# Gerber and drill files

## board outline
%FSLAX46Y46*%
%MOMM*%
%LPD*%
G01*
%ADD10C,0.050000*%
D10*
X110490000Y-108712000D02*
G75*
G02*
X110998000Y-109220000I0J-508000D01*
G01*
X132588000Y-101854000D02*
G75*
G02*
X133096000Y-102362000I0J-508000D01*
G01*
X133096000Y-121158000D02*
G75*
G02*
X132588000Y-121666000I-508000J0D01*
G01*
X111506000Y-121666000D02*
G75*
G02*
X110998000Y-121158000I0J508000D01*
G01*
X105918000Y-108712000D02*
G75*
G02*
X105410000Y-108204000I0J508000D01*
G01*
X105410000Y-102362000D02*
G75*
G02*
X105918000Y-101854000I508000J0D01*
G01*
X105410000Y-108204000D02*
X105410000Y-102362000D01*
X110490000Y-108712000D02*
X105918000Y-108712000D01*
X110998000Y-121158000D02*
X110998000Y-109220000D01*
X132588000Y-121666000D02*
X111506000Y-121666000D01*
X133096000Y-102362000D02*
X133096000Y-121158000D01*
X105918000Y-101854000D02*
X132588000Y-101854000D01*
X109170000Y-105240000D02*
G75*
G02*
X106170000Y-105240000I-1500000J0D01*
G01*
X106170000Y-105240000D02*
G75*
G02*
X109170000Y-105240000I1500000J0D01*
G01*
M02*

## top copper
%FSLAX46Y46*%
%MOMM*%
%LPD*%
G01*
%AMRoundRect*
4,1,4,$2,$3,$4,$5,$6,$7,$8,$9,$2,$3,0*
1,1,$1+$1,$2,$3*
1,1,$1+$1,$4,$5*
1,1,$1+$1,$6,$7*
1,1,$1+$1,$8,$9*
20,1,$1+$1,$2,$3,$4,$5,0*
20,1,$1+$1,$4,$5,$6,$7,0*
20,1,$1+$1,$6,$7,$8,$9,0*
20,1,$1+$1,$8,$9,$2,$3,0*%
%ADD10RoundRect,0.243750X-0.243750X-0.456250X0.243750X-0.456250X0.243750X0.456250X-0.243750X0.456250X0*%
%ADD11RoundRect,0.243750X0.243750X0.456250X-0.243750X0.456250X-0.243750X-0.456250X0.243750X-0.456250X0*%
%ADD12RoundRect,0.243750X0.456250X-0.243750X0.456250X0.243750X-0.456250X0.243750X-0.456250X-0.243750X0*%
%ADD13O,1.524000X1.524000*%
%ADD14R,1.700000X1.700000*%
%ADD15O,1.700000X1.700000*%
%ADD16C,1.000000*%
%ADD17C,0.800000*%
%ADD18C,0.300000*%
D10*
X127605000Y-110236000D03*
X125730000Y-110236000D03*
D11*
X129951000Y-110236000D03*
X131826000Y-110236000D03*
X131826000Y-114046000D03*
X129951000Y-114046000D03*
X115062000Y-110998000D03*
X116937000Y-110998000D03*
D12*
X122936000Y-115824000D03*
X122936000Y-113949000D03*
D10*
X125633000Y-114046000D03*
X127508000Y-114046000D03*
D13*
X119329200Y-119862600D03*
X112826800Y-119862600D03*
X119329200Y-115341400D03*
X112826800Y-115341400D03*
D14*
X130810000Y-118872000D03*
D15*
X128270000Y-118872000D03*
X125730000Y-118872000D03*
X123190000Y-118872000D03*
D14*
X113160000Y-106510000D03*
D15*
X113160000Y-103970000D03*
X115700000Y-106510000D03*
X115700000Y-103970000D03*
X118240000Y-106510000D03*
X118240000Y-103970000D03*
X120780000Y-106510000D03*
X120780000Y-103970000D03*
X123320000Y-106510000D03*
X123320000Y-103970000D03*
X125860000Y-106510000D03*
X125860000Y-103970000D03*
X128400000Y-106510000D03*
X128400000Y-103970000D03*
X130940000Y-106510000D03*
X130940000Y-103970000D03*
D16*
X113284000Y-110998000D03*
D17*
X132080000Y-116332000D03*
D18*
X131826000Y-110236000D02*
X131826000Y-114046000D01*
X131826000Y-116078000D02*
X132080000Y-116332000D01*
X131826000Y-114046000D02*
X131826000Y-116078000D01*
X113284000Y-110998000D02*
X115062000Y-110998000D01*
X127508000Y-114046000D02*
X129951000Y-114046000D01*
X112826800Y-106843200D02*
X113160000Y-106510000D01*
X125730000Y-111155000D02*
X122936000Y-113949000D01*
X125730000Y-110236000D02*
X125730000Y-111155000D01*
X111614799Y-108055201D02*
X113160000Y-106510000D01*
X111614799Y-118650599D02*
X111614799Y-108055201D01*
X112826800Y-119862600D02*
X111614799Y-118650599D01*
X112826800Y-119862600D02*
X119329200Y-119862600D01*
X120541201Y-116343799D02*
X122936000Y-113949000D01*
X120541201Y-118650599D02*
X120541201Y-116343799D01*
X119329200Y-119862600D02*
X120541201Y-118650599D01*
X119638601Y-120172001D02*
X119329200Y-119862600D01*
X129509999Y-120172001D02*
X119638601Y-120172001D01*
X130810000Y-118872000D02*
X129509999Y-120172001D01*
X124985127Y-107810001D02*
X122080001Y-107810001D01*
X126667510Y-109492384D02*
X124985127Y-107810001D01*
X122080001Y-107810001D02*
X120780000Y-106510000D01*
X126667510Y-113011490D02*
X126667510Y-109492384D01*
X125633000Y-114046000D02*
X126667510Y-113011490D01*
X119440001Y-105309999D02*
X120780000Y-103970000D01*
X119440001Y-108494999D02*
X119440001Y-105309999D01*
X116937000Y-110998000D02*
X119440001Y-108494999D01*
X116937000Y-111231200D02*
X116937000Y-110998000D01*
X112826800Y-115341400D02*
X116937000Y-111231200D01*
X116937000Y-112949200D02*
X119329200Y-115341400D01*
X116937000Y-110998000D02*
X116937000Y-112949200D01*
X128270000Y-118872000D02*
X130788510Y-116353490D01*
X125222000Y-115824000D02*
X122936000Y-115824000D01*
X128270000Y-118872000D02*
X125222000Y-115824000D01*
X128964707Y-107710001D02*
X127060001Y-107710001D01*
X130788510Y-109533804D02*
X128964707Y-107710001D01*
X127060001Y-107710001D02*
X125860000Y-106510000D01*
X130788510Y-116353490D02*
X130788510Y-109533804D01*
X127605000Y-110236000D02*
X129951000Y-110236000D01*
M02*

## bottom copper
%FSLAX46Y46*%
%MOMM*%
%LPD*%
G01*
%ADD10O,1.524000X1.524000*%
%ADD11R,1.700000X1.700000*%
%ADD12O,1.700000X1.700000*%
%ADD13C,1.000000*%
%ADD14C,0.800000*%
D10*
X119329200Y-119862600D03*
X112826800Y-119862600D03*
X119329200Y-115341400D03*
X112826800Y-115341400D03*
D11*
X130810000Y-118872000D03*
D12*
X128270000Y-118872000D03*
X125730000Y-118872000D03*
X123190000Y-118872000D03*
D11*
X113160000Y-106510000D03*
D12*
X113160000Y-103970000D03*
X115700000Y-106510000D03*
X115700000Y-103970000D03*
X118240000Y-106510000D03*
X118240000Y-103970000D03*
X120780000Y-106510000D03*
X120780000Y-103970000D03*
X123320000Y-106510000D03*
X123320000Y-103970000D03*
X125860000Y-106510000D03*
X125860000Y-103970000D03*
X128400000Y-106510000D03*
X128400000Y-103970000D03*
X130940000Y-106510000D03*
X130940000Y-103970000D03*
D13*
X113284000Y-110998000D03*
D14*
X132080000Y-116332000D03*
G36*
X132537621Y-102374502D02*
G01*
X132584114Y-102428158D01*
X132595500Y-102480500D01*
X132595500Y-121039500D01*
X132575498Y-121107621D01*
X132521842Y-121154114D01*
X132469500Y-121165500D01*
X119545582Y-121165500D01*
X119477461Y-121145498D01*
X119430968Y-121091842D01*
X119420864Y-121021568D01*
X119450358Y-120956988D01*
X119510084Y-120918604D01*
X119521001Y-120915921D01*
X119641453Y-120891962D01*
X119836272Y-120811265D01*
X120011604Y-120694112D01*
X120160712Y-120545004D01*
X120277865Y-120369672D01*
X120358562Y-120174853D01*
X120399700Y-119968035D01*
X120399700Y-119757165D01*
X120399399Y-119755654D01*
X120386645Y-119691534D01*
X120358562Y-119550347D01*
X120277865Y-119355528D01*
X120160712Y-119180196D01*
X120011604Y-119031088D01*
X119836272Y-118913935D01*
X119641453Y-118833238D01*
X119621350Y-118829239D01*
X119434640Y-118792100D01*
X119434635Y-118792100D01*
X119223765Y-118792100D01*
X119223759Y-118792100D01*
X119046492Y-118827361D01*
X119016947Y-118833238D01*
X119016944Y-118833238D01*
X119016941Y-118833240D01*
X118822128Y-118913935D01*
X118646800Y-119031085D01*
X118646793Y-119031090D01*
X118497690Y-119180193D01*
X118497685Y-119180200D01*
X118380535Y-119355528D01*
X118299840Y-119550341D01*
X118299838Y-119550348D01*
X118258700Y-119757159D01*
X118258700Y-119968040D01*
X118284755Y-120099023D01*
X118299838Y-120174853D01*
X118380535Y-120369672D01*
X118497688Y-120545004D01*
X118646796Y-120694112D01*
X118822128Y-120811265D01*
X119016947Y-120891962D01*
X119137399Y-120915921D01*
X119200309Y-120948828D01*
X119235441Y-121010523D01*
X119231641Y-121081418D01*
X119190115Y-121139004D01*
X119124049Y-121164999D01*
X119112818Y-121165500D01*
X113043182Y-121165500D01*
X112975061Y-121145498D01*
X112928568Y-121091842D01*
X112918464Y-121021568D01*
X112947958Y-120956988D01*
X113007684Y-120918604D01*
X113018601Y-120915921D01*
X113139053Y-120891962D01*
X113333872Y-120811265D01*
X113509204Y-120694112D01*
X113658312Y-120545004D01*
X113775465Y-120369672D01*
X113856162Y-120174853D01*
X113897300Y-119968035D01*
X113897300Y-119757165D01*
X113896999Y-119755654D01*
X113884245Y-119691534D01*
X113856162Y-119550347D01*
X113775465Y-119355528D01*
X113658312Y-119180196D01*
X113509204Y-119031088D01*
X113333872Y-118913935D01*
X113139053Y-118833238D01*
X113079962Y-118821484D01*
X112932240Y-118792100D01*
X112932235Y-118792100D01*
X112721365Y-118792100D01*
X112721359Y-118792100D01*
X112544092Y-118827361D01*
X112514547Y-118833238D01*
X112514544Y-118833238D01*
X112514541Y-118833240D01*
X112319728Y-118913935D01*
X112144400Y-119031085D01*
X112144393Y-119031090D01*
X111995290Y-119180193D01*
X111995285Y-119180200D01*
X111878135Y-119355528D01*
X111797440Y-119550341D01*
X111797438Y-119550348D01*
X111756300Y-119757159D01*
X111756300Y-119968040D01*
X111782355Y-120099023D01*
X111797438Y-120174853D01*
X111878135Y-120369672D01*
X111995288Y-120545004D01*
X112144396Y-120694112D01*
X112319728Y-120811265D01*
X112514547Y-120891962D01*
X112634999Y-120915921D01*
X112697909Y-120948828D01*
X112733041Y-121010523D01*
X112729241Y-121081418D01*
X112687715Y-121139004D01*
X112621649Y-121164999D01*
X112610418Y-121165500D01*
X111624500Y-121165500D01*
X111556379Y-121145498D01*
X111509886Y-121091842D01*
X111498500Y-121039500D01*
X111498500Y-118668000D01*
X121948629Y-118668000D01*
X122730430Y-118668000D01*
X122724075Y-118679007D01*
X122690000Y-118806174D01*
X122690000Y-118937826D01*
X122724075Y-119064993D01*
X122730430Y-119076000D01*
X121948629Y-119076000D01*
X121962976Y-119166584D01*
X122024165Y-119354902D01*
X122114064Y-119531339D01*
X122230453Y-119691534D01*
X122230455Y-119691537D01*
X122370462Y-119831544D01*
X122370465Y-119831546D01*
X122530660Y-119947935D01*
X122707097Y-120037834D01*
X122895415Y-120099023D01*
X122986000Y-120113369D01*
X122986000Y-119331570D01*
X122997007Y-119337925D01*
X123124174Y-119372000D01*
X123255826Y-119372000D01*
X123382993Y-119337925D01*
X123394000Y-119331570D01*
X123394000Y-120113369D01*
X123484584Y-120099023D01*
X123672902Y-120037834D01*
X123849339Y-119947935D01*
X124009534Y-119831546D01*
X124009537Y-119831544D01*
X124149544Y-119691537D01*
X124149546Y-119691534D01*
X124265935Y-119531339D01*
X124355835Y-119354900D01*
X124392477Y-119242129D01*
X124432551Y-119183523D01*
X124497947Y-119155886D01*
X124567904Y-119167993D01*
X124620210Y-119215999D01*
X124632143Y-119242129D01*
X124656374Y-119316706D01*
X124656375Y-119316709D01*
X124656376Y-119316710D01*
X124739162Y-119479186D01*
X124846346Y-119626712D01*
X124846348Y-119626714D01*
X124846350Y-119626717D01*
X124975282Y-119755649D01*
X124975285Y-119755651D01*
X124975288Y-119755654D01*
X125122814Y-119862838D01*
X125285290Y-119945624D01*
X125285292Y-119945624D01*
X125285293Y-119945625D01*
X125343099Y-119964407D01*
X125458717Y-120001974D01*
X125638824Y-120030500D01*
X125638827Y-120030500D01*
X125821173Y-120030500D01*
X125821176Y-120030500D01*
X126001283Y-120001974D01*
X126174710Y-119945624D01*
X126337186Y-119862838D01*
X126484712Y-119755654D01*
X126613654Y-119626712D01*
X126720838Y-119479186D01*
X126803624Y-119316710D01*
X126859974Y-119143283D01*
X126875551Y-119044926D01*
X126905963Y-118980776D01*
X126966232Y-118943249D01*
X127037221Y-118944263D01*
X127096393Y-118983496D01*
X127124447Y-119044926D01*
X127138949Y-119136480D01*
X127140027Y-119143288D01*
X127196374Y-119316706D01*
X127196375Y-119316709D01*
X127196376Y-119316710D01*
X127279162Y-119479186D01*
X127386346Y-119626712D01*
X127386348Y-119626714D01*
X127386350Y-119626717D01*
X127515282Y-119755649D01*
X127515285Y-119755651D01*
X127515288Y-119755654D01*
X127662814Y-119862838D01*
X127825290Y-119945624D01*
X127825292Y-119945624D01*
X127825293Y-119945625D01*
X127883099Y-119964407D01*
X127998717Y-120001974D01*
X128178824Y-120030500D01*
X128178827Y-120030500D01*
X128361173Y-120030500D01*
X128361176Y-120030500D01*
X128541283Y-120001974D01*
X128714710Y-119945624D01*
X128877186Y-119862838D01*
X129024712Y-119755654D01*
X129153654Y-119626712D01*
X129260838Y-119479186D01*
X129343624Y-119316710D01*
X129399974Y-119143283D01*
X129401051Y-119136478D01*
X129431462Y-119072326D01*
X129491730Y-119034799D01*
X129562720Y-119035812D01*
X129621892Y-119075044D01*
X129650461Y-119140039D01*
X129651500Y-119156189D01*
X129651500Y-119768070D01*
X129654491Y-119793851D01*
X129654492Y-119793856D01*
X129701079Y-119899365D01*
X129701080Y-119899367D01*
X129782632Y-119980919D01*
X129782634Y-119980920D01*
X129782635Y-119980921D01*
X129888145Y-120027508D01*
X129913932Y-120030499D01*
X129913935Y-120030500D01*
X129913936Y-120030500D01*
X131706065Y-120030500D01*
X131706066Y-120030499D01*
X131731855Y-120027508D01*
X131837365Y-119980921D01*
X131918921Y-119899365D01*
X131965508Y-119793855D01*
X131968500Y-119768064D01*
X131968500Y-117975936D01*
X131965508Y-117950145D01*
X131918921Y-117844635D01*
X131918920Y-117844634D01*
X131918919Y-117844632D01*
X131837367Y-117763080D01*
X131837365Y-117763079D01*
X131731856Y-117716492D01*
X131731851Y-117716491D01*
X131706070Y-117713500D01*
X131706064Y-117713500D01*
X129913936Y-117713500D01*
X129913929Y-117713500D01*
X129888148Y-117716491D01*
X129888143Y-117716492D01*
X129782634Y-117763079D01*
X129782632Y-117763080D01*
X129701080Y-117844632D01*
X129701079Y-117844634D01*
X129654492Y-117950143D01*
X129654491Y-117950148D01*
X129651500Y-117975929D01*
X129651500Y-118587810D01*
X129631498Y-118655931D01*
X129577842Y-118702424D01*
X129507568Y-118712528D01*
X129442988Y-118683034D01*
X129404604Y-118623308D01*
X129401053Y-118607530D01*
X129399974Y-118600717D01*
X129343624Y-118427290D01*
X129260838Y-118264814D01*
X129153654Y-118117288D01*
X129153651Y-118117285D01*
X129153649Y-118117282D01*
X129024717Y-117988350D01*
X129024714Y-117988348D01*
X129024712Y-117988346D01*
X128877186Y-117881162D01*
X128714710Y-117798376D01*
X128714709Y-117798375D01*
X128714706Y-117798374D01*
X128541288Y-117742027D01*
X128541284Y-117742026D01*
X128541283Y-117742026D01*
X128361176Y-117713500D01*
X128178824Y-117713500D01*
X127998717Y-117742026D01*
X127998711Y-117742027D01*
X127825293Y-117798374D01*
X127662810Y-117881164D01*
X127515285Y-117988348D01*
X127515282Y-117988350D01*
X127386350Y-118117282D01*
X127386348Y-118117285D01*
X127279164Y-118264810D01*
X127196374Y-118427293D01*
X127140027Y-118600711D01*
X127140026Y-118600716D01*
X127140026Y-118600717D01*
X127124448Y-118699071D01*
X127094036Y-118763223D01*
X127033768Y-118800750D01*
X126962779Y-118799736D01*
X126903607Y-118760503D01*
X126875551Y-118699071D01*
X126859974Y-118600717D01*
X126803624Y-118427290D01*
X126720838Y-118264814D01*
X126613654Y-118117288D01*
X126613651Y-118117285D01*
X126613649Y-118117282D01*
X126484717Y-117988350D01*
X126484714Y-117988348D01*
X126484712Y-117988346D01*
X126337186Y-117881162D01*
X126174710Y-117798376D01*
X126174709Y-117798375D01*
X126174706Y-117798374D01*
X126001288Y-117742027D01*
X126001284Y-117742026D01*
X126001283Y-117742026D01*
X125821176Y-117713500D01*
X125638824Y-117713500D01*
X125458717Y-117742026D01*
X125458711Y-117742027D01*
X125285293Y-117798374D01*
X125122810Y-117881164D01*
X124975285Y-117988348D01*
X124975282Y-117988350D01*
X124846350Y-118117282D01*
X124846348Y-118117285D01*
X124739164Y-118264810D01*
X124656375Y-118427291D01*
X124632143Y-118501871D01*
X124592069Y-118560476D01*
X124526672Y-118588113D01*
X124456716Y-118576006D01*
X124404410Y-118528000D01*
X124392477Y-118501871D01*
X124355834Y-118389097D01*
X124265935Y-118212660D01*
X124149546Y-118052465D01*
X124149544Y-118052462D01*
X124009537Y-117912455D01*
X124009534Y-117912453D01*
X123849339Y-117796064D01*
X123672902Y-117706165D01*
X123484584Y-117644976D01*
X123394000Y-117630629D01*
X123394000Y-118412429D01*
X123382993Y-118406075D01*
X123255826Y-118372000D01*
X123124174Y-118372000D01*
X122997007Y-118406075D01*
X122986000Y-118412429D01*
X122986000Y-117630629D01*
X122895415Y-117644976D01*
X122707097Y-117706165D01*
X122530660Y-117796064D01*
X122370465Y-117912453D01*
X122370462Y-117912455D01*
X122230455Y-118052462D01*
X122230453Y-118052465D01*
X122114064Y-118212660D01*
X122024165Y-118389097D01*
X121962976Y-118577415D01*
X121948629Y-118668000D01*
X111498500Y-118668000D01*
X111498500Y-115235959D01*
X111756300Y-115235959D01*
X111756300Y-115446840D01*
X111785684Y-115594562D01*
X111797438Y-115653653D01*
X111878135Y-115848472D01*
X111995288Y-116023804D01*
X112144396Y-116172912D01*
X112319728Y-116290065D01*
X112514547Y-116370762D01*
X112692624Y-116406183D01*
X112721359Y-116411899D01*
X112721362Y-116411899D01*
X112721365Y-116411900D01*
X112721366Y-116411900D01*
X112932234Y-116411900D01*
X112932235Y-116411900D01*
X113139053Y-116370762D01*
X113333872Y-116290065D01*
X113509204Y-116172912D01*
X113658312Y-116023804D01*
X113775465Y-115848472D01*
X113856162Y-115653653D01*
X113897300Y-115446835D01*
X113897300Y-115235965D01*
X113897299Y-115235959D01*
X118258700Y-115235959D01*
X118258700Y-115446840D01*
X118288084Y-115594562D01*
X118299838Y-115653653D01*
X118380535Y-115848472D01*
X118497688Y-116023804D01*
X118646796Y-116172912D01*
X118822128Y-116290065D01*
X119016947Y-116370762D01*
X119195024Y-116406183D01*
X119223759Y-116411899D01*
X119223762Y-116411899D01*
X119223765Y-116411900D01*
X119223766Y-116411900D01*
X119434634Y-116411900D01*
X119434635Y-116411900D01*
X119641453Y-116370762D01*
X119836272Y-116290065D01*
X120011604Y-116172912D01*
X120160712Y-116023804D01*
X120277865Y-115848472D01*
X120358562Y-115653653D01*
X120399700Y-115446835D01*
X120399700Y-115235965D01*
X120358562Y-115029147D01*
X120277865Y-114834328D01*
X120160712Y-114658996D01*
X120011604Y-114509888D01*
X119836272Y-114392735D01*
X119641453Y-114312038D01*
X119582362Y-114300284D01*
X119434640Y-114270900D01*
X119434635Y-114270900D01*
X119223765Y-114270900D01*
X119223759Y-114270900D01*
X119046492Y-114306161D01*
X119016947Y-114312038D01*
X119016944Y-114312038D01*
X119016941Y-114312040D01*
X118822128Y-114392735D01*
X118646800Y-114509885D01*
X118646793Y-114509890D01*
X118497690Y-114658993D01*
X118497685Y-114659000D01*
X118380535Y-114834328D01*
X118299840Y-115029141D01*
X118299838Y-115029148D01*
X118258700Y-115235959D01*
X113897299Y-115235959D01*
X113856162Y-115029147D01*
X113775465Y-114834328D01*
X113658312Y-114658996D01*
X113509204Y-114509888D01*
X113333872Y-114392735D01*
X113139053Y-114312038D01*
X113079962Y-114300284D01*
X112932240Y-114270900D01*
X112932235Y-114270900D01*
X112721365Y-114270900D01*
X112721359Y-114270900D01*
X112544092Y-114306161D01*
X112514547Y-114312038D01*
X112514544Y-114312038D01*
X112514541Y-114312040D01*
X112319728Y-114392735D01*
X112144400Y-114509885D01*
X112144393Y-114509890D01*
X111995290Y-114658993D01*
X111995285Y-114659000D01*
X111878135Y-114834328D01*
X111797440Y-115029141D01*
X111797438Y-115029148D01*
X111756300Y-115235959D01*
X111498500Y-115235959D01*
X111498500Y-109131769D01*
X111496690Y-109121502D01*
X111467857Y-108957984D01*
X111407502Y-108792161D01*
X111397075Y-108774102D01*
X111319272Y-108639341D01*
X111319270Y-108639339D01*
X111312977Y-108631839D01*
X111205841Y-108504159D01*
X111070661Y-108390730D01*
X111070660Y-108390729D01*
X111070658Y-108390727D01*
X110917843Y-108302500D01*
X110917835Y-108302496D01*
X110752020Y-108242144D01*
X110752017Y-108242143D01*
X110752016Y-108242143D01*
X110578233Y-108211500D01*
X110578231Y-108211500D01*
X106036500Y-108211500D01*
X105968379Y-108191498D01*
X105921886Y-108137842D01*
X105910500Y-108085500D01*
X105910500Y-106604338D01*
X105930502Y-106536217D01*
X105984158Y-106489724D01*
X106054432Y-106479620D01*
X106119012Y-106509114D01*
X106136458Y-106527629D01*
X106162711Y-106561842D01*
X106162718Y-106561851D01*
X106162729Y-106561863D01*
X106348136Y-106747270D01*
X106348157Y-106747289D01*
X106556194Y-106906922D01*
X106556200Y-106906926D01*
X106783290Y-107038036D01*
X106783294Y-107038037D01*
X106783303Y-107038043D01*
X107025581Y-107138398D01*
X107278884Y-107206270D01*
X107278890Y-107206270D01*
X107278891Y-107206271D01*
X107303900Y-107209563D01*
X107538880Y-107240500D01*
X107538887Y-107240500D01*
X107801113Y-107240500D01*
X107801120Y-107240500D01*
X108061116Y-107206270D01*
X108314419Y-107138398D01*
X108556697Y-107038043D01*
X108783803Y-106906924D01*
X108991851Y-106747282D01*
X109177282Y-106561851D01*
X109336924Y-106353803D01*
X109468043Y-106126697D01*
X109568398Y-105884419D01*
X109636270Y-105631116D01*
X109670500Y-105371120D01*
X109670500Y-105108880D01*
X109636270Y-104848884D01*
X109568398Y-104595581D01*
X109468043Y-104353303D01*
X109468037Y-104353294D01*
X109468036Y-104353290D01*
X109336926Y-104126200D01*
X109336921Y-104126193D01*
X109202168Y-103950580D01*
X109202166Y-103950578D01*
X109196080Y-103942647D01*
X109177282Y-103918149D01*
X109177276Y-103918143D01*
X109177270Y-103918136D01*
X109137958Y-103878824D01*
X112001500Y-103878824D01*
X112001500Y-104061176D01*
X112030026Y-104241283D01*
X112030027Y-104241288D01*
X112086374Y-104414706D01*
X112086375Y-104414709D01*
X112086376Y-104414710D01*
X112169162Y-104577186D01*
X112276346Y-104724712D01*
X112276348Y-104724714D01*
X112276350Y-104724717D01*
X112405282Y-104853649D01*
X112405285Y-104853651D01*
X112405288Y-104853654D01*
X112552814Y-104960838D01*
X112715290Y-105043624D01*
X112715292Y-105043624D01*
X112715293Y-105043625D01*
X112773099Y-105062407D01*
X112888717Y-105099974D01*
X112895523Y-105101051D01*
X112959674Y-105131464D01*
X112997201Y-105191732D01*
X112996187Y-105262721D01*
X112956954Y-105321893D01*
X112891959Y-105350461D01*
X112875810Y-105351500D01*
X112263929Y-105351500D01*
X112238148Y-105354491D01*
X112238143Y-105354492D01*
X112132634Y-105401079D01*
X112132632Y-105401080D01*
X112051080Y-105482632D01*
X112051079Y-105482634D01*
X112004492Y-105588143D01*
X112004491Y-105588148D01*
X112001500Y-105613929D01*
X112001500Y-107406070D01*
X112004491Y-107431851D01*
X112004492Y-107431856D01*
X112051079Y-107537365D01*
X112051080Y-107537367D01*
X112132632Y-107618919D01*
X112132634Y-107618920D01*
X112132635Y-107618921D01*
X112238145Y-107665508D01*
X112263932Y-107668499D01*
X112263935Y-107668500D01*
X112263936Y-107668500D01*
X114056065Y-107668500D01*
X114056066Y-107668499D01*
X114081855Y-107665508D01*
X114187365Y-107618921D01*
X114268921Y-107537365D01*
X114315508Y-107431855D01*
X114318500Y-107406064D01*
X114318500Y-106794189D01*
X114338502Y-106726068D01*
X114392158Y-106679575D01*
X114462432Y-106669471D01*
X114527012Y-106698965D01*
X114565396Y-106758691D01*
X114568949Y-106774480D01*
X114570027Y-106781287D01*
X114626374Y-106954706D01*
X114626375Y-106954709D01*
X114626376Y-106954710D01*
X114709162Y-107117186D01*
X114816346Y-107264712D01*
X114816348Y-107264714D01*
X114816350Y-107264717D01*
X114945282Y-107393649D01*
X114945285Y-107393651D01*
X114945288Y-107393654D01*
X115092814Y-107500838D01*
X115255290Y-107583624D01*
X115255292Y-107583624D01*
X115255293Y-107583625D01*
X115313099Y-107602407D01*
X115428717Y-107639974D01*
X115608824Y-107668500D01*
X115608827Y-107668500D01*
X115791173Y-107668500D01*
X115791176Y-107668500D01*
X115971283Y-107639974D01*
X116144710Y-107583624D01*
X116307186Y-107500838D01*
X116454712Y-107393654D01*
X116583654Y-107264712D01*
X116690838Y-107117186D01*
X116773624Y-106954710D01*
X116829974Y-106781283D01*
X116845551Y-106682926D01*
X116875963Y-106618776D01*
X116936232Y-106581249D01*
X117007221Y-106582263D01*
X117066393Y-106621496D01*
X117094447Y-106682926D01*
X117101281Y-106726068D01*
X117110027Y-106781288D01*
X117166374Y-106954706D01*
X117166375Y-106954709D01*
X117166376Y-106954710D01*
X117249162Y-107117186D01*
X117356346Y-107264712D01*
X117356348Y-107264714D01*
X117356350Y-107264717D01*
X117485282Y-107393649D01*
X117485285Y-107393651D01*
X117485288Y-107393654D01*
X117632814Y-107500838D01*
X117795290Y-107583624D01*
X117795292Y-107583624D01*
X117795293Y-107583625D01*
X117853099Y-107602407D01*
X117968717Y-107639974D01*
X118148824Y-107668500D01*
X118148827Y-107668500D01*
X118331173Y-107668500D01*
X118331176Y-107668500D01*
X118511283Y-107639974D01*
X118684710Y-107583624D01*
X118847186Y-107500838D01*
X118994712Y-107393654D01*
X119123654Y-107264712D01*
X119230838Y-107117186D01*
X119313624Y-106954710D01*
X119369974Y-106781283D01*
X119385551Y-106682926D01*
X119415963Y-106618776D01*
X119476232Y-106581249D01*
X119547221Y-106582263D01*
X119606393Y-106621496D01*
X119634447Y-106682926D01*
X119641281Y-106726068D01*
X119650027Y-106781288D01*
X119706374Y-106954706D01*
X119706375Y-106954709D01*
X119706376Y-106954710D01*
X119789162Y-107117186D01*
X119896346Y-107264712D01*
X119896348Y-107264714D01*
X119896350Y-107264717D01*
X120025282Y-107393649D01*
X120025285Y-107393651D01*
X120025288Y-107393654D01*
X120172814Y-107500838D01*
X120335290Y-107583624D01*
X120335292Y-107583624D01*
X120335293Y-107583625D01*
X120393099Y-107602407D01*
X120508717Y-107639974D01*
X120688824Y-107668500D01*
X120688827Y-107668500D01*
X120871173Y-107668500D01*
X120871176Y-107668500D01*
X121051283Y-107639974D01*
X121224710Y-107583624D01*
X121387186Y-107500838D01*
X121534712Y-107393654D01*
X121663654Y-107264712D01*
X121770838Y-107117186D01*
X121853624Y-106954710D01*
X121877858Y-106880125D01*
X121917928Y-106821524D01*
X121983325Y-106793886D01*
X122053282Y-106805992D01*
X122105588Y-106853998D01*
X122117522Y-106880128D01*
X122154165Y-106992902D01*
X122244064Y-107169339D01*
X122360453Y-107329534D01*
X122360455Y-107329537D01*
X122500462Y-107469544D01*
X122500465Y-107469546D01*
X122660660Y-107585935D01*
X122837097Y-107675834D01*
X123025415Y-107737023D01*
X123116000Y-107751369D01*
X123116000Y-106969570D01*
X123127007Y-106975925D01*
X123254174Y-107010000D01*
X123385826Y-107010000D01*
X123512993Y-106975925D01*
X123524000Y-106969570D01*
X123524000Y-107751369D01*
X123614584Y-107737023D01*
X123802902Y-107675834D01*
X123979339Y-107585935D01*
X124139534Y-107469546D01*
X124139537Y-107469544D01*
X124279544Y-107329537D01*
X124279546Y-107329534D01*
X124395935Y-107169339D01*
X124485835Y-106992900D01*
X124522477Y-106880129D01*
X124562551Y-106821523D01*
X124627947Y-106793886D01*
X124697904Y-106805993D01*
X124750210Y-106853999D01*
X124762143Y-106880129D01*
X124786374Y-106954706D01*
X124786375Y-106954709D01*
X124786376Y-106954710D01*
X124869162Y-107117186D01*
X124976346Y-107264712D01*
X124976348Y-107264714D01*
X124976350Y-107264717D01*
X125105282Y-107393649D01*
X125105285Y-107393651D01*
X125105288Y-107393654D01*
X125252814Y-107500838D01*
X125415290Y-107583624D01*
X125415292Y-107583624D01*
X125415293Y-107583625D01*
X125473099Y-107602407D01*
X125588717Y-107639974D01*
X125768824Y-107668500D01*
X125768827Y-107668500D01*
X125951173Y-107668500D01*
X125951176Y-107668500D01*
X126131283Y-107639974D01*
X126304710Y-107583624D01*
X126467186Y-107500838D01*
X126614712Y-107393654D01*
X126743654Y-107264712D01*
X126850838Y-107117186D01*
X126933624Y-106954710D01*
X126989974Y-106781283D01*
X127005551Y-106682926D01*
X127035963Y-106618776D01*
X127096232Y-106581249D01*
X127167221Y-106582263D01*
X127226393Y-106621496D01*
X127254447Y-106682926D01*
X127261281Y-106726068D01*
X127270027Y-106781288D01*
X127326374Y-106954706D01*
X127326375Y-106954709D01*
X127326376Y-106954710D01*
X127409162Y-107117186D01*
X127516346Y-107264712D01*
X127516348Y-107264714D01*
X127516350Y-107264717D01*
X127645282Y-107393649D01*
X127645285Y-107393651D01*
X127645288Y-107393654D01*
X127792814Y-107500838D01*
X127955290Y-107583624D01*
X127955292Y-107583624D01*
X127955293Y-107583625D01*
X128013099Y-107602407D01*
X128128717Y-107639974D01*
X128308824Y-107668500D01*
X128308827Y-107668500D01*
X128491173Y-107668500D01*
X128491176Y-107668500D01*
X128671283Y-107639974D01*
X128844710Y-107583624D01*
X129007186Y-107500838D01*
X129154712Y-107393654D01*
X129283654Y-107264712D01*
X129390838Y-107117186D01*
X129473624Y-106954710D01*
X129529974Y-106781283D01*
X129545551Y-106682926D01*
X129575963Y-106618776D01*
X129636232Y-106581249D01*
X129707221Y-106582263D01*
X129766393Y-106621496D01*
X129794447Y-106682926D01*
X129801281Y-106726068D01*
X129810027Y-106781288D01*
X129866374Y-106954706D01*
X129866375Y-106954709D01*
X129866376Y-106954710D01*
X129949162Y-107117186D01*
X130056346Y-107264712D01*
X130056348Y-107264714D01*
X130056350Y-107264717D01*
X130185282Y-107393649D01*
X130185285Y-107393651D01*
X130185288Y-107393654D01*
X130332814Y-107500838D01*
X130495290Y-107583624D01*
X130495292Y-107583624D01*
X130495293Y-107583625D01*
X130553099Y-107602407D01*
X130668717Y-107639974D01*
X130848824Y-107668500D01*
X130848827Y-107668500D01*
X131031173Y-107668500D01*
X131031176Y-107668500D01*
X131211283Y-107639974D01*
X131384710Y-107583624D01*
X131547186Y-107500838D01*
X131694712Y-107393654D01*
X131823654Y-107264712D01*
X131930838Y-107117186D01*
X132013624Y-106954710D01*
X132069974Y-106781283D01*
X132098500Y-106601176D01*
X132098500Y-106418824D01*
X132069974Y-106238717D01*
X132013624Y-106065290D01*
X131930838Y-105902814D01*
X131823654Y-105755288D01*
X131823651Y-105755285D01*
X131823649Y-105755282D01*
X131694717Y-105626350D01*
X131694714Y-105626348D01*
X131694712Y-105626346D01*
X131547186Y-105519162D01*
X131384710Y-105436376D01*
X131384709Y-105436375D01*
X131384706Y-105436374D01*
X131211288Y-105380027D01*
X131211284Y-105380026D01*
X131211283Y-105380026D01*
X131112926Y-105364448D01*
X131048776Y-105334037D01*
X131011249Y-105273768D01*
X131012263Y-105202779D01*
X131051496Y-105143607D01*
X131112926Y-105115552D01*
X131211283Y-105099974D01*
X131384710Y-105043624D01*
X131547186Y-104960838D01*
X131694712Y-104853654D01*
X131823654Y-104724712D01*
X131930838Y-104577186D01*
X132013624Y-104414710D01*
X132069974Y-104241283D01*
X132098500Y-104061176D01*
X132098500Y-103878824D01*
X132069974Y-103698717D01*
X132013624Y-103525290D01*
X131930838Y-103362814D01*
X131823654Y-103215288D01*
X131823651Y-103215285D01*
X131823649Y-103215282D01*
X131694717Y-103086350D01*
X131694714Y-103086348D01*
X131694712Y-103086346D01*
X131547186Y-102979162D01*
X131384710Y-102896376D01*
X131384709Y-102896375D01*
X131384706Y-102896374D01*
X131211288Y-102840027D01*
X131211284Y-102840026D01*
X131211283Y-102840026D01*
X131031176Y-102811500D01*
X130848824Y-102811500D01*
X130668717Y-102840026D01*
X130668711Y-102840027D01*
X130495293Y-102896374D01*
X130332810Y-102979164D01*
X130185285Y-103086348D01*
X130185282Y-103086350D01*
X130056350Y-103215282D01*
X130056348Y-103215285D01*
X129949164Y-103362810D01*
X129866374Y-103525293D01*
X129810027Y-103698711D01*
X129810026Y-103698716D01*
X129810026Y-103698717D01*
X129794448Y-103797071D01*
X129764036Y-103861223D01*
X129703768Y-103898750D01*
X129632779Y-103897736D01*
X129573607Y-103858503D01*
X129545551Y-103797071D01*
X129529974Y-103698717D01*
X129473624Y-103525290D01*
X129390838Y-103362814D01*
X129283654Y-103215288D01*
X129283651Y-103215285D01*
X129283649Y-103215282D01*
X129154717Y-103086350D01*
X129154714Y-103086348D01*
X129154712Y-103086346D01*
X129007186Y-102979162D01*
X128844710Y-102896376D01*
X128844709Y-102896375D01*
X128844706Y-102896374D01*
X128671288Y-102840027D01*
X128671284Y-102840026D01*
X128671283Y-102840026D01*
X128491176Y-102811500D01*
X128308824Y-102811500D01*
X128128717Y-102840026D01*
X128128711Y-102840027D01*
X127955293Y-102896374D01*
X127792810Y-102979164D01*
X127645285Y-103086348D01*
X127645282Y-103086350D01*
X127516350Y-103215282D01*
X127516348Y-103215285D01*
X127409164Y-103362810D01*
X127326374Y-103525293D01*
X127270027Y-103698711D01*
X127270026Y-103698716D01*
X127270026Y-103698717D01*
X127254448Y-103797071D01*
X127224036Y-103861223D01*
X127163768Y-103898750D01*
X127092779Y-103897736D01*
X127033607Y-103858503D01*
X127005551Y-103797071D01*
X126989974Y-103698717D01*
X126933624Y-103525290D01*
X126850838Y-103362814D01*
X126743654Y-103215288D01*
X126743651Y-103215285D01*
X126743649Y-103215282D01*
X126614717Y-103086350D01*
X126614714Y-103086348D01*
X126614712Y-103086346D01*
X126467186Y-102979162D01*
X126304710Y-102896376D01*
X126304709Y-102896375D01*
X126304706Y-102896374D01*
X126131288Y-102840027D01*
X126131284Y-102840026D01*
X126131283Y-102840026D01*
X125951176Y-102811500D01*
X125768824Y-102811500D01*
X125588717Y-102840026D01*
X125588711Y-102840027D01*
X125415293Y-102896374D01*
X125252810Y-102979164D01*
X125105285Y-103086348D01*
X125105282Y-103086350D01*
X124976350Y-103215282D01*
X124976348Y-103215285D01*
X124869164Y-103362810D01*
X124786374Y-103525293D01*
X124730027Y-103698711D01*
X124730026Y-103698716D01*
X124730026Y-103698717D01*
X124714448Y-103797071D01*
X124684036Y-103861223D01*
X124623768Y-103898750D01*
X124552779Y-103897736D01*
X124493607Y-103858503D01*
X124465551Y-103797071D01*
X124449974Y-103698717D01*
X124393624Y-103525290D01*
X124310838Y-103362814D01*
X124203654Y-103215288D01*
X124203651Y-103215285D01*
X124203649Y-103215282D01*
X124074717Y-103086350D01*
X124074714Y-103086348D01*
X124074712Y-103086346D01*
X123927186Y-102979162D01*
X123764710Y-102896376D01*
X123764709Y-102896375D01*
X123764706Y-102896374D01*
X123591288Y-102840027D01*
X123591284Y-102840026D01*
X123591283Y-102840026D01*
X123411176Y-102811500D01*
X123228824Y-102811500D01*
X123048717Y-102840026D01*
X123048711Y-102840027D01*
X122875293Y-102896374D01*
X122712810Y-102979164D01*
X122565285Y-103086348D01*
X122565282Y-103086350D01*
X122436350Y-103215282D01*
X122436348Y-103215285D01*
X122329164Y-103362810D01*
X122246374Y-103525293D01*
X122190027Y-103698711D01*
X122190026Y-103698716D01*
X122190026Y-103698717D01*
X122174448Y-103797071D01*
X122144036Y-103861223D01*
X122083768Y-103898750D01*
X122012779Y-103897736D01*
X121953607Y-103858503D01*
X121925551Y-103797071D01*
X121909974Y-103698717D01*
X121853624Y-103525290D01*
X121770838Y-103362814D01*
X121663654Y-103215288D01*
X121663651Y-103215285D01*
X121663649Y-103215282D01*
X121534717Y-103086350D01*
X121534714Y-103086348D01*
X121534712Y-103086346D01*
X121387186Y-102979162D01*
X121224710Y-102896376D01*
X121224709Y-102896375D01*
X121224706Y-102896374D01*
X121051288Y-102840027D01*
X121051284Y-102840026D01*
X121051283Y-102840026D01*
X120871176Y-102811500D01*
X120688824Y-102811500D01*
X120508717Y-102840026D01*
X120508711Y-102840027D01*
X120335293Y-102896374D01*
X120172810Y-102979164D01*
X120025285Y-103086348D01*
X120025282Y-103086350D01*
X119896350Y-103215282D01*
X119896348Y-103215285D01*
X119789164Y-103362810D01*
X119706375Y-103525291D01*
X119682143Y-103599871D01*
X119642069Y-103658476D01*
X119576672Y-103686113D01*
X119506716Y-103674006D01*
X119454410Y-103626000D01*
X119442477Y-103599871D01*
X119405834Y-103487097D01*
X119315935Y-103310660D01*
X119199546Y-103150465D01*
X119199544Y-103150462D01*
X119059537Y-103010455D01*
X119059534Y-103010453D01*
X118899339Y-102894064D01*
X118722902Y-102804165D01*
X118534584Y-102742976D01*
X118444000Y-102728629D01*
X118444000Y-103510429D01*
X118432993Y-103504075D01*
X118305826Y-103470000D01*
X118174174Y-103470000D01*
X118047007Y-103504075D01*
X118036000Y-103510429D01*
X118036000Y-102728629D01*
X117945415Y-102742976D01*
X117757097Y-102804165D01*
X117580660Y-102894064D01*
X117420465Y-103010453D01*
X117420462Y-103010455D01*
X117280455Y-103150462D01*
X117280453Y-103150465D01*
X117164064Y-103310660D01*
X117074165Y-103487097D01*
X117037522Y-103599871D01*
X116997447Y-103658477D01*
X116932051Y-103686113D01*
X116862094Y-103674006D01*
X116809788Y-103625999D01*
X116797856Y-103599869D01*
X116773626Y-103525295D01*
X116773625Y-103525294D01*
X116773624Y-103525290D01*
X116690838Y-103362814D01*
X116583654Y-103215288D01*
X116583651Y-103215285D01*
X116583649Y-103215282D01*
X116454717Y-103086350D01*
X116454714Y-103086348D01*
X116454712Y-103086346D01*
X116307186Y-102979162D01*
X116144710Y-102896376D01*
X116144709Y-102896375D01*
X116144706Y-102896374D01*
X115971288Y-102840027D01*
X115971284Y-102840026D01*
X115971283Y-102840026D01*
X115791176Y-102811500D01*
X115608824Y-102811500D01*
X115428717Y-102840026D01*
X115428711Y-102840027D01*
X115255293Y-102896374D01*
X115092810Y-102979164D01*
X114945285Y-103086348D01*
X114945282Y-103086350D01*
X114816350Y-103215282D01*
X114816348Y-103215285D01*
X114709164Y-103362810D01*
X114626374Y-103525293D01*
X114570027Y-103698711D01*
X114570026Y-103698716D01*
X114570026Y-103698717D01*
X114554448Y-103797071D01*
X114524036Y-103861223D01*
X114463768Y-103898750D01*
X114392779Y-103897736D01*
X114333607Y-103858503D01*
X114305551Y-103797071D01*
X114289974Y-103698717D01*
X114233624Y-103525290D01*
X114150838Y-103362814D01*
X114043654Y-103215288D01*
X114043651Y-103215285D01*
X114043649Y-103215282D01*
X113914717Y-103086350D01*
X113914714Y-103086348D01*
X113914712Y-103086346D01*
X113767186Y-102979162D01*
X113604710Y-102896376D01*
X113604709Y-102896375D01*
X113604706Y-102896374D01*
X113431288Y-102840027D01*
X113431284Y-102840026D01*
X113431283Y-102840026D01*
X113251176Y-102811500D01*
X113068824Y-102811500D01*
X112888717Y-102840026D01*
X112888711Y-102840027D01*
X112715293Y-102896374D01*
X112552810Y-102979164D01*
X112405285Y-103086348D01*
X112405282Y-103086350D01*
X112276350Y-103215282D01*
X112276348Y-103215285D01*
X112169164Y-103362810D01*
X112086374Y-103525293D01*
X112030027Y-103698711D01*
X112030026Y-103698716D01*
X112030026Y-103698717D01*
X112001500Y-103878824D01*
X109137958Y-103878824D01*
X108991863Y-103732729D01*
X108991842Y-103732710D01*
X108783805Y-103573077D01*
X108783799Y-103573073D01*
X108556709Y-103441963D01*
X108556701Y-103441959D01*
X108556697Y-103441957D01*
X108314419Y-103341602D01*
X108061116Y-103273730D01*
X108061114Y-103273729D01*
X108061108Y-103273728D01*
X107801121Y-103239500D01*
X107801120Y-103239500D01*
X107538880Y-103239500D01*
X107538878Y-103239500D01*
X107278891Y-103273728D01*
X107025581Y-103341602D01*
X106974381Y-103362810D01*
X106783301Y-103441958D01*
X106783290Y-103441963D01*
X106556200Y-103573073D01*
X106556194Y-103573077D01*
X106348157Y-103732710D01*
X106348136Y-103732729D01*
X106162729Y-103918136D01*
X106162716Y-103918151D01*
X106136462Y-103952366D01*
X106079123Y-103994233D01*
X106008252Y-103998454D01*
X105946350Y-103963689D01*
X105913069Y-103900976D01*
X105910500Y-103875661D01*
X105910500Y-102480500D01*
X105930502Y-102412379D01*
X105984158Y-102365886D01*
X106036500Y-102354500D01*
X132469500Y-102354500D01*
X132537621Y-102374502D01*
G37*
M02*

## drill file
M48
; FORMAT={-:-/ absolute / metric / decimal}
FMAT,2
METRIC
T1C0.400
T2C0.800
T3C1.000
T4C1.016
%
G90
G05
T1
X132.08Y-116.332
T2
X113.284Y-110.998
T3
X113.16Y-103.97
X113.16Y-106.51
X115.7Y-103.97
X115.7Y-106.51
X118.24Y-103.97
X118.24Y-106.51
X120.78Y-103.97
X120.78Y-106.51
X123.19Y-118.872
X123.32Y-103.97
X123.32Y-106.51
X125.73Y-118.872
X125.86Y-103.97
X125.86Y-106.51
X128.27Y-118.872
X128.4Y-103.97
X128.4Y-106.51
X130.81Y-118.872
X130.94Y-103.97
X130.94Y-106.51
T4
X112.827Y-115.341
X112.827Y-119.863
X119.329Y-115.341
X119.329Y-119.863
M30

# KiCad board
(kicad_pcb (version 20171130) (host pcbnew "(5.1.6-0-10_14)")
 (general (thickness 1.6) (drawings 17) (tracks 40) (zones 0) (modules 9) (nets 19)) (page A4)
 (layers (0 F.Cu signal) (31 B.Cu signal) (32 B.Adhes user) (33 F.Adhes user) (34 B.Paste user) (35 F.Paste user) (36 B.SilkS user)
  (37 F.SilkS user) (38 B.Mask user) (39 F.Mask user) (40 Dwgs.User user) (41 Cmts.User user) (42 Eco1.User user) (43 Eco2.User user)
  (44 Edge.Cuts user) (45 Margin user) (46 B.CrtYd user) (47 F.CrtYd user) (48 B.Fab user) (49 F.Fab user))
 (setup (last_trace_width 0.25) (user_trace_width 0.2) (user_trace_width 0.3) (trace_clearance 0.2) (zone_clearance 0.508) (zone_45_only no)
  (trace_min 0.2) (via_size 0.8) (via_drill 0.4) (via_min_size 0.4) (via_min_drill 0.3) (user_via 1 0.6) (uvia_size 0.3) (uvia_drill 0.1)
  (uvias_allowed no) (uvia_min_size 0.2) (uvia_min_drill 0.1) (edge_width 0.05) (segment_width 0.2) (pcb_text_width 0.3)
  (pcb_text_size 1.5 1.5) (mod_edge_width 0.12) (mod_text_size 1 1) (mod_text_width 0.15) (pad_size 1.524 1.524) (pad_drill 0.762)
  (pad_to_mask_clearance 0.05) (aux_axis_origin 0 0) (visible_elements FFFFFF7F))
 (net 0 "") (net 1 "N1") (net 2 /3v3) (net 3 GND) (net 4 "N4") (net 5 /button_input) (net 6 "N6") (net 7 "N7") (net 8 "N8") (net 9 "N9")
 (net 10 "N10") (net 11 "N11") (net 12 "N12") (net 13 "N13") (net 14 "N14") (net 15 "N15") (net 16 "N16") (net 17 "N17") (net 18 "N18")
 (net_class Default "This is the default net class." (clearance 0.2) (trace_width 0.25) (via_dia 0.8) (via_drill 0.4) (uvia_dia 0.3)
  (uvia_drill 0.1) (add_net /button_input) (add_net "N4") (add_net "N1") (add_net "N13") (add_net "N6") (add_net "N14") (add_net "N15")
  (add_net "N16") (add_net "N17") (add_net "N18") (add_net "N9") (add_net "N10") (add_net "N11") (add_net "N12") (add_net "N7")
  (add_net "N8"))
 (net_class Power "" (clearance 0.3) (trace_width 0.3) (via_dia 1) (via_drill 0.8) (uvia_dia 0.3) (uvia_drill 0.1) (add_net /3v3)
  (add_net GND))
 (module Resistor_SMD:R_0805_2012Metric (layer F.Cu) (at 126.6675 110.236)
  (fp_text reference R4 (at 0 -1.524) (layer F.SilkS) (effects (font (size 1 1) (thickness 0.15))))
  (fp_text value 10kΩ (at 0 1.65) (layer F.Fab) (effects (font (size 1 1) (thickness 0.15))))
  (pad 2 smd roundrect (at 0.9375 0) (size 0.975 1.4) (layers F.Cu F.Paste F.Mask) (roundrect_rratio 0.25) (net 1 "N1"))
  (pad 1 smd roundrect (at -0.9375 0) (size 0.975 1.4) (layers F.Cu F.Paste F.Mask) (roundrect_rratio 0.25) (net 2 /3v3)))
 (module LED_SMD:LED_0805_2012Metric (layer F.Cu) (at 130.8885 110.236 180)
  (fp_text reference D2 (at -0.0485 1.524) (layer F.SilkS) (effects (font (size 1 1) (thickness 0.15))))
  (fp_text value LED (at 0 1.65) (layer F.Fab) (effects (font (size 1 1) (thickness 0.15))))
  (pad 2 smd roundrect (at 0.9375 0 180) (size 0.975 1.4) (layers F.Cu F.Paste F.Mask) (roundrect_rratio 0.25) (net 1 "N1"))
  (pad 1 smd roundrect (at -0.9375 0 180) (size 0.975 1.4) (layers F.Cu F.Paste F.Mask) (roundrect_rratio 0.25) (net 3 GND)))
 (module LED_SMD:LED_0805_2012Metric (layer F.Cu) (at 130.8885 114.046 180)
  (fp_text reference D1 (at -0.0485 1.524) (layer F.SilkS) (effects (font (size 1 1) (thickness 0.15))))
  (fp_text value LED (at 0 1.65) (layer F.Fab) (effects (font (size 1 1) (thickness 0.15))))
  (pad 1 smd roundrect (at -0.9375 0 180) (size 0.975 1.4) (layers F.Cu F.Paste F.Mask) (roundrect_rratio 0.25) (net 3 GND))
  (pad 2 smd roundrect (at 0.9375 0 180) (size 0.975 1.4) (layers F.Cu F.Paste F.Mask) (roundrect_rratio 0.25) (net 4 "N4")))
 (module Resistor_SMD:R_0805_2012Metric (layer F.Cu) (at 115.9995 110.998 180)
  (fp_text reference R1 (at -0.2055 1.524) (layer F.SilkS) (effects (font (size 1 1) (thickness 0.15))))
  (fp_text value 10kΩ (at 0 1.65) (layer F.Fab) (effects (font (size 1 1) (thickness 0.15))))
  (pad 2 smd roundrect (at 0.9375 0 180) (size 0.975 1.4) (layers F.Cu F.Paste F.Mask) (roundrect_rratio 0.25) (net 3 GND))
  (pad 1 smd roundrect (at -0.9375 0 180) (size 0.975 1.4) (layers F.Cu F.Paste F.Mask) (roundrect_rratio 0.25) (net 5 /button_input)))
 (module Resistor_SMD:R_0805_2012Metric (layer F.Cu) (at 122.936 114.8865 90)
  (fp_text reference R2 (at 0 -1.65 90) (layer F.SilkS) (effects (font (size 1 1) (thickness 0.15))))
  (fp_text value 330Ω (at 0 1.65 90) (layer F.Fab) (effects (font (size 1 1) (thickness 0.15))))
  (pad 1 smd roundrect (at -0.9375 0 90) (size 0.975 1.4) (layers F.Cu F.Paste F.Mask) (roundrect_rratio 0.25) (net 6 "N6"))
  (pad 2 smd roundrect (at 0.9375 0 90) (size 0.975 1.4) (layers F.Cu F.Paste F.Mask) (roundrect_rratio 0.25) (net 2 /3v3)))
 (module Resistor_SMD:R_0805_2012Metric (layer F.Cu) (at 126.5705 114.046)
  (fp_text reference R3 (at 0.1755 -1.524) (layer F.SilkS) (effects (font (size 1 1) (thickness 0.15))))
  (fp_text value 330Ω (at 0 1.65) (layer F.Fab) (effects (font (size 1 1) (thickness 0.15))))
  (pad 1 smd roundrect (at -0.9375 0) (size 0.975 1.4) (layers F.Cu F.Paste F.Mask) (roundrect_rratio 0.25) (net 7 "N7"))
  (pad 2 smd roundrect (at 0.9375 0) (size 0.975 1.4) (layers F.Cu F.Paste F.Mask) (roundrect_rratio 0.25) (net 4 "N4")))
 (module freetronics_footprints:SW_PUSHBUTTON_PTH (layer F.Cu) (at 116.078 117.602 180)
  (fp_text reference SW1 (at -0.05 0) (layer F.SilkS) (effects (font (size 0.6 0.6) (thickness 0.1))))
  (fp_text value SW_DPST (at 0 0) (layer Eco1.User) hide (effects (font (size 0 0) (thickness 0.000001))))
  (pad 1 thru_hole oval (at -3.2512 -2.2606 180) (size 1.524 1.524) (drill 1.016) (layers *.Cu *.Mask) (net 2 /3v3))
  (pad 1 thru_hole oval (at 3.2512 -2.2606 180) (size 1.524 1.524) (drill 1.016) (layers *.Cu *.Mask) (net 2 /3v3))
  (pad 2 thru_hole oval (at -3.2512 2.2606 180) (size 1.524 1.524) (drill 1.016) (layers *.Cu *.Mask) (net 5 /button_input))
  (pad 2 thru_hole oval (at 3.2512 2.2606 180) (size 1.524 1.524) (drill 1.016) (layers *.Cu *.Mask) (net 5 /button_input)))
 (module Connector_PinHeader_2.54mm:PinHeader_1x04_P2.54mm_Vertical (layer F.Cu) (at 130.81 118.872 270)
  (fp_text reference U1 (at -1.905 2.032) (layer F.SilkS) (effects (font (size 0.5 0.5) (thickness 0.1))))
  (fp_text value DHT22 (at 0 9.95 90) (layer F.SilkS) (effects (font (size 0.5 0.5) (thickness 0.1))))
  (pad 1 thru_hole rect (at 0 0 270) (size 1.7 1.7) (drill 1) (layers *.Cu *.Mask) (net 2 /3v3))
  (pad 2 thru_hole oval (at 0 2.54 270) (size 1.7 1.7) (drill 1) (layers *.Cu *.Mask) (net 6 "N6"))
  (pad 3 thru_hole oval (at 0 5.08 270) (size 1.7 1.7) (drill 1) (layers *.Cu *.Mask) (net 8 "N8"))
  (pad 4 thru_hole oval (at 0 7.62 270) (size 1.7 1.7) (drill 1) (layers *.Cu *.Mask) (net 3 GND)))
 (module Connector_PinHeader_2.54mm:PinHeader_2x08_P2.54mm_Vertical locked (layer F.Cu) (at 113.16 106.51 90)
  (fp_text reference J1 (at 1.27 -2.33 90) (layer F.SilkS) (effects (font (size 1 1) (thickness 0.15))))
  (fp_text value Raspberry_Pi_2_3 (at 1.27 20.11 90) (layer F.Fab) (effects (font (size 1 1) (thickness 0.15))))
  (pad 1 thru_hole rect (at 0 0 90) (size 1.7 1.7) (drill 1) (layers *.Cu *.Mask) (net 2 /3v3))
  (pad 2 thru_hole oval (at 2.54 0 90) (size 1.7 1.7) (drill 1) (layers *.Cu *.Mask) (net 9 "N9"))
  (pad 3 thru_hole oval (at 0 2.54 90) (size 1.7 1.7) (drill 1) (layers *.Cu *.Mask) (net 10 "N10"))
  (pad 4 thru_hole oval (at 2.54 2.54 90) (size 1.7 1.7) (drill 1) (layers *.Cu *.Mask) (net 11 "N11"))
  (pad 5 thru_hole oval (at 0 5.08 90) (size 1.7 1.7) (drill 1) (layers *.Cu *.Mask) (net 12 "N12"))
  (pad 6 thru_hole oval (at 2.54 5.08 90) (size 1.7 1.7) (drill 1) (layers *.Cu *.Mask) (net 3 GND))
  (pad 7 thru_hole oval (at 0 7.62 90) (size 1.7 1.7) (drill 1) (layers *.Cu *.Mask) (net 7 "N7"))
  (pad 8 thru_hole oval (at 2.54 7.62 90) (size 1.7 1.7) (drill 1) (layers *.Cu *.Mask) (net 5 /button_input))
  (pad 9 thru_hole oval (at 0 10.16 90) (size 1.7 1.7) (drill 1) (layers *.Cu *.Mask) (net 3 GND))
  (pad 10 thru_hole oval (at 2.54 10.16 90) (size 1.7 1.7) (drill 1) (layers *.Cu *.Mask) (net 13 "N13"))
  (pad 11 thru_hole oval (at 0 12.7 90) (size 1.7 1.7) (drill 1) (layers *.Cu *.Mask) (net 6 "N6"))
  (pad 12 thru_hole oval (at 2.54 12.7 90) (size 1.7 1.7) (drill 1) (layers *.Cu *.Mask) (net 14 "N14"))
  (pad 13 thru_hole oval (at 0 15.24 90) (size 1.7 1.7) (drill 1) (layers *.Cu *.Mask) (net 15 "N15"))
  (pad 14 thru_hole oval (at 2.54 15.24 90) (size 1.7 1.7) (drill 1) (layers *.Cu *.Mask) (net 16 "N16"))
  (pad 15 thru_hole oval (at 0 17.78 90) (size 1.7 1.7) (drill 1) (layers *.Cu *.Mask) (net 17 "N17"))
  (pad 16 thru_hole oval (at 2.54 17.78 90) (size 1.7 1.7) (drill 1) (layers *.Cu *.Mask) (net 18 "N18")))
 (gr_arc (start 110.49 109.22) (end 110.998 109.22) (angle -90) (layer Edge.Cuts) (width 0.05))
 (gr_arc (start 132.588 102.362) (end 133.096 102.362) (angle -90) (layer Edge.Cuts) (width 0.05))
 (gr_arc (start 132.588 121.158) (end 132.588 121.666) (angle -90) (layer Edge.Cuts) (width 0.05))
 (gr_arc (start 111.506 121.158) (end 110.998 121.158) (angle -90) (layer Edge.Cuts) (width 0.05))
 (gr_arc (start 105.918 108.204) (end 105.41 108.204) (angle -90) (layer Edge.Cuts) (width 0.05))
 (gr_arc (start 105.918 102.362) (end 105.918 101.854) (angle -90) (layer Edge.Cuts) (width 0.05))
 (gr_line (start 105.41 108.204) (end 105.41 102.362) (layer Edge.Cuts) (width 0.05))
 (gr_line (start 110.49 108.712) (end 105.918 108.712) (layer Edge.Cuts) (width 0.05))
 (gr_line (start 110.998 121.158) (end 110.998 109.22) (layer Edge.Cuts) (width 0.05))
 (gr_line (start 132.588 121.666) (end 111.506 121.666) (layer Edge.Cuts) (width 0.05))
 (gr_line (start 133.096 102.362) (end 133.096 121.158) (layer Edge.Cuts) (width 0.05))
 (gr_line (start 105.918 101.854) (end 132.588 101.854) (layer Edge.Cuts) (width 0.05))
 (gr_circle (center 107.67 105.24) (end 106.17 105.24) (layer Edge.Cuts) (width 0.05))
 (via (at 113.284 110.998) (size 1) (drill 0.8) (layers F.Cu B.Cu) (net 3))
 (via (at 132.08 116.332) (size 0.8) (drill 0.4) (layers F.Cu B.Cu) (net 3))
 (segment (start 131.826 110.236) (end 131.826 114.046) (width 0.3) (layer F.Cu) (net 3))
 (segment (start 131.826 116.078) (end 132.08 116.332) (width 0.3) (layer F.Cu) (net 3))
 (segment (start 131.826 114.046) (end 131.826 116.078) (width 0.3) (layer F.Cu) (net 3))
 (segment (start 113.284 110.998) (end 115.062 110.998) (width 0.3) (layer F.Cu) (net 3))
 (segment (start 127.508 114.046) (end 129.951 114.046) (width 0.3) (layer F.Cu) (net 4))
 (segment (start 112.8268 106.8432) (end 113.16 106.51) (width 0.3) (layer F.Cu) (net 2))
 (segment (start 125.73 111.155) (end 122.936 113.949) (width 0.3) (layer F.Cu) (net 2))
 (segment (start 125.73 110.236) (end 125.73 111.155) (width 0.3) (layer F.Cu) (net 2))
 (segment (start 111.614799 108.055201) (end 113.16 106.51) (width 0.3) (layer F.Cu) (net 2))
 (segment (start 111.614799 118.650599) (end 111.614799 108.055201) (width 0.3) (layer F.Cu) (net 2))
 (segment (start 112.8268 119.8626) (end 111.614799 118.650599) (width 0.3) (layer F.Cu) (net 2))
 (segment (start 112.8268 119.8626) (end 119.3292 119.8626) (width 0.3) (layer F.Cu) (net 2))
 (segment (start 120.541201 116.343799) (end 122.936 113.949) (width 0.3) (layer F.Cu) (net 2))
 (segment (start 120.541201 118.650599) (end 120.541201 116.343799) (width 0.3) (layer F.Cu) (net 2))
 (segment (start 119.3292 119.8626) (end 120.541201 118.650599) (width 0.3) (layer F.Cu) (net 2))
 (segment (start 119.638601 120.172001) (end 119.3292 119.8626) (width 0.3) (layer F.Cu) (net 2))
 (segment (start 129.509999 120.172001) (end 119.638601 120.172001) (width 0.3) (layer F.Cu) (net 2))
 (segment (start 130.81 118.872) (end 129.509999 120.172001) (width 0.3) (layer F.Cu) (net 2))
 (segment (start 124.985127 107.810001) (end 122.080001 107.810001) (width 0.3) (layer F.Cu) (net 7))
 (segment (start 126.66751 109.492384) (end 124.985127 107.810001) (width 0.3) (layer F.Cu) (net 7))
 (segment (start 122.080001 107.810001) (end 120.78 106.51) (width 0.3) (layer F.Cu) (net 7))
 (segment (start 126.66751 113.01149) (end 126.66751 109.492384) (width 0.3) (layer F.Cu) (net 7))
 (segment (start 125.633 114.046) (end 126.66751 113.01149) (width 0.3) (layer F.Cu) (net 7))
 (segment (start 119.440001 105.309999) (end 120.78 103.97) (width 0.3) (layer F.Cu) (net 5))
 (segment (start 119.440001 108.494999) (end 119.440001 105.309999) (width 0.3) (layer F.Cu) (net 5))
 (segment (start 116.937 110.998) (end 119.440001 108.494999) (width 0.3) (layer F.Cu) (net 5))
 (segment (start 116.937 111.2312) (end 116.937 110.998) (width 0.3) (layer F.Cu) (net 5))
 (segment (start 112.8268 115.3414) (end 116.937 111.2312) (width 0.3) (layer F.Cu) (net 5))
 (segment (start 116.937 112.9492) (end 119.3292 115.3414) (width 0.3) (layer F.Cu) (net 5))
 (segment (start 116.937 110.998) (end 116.937 112.9492) (width 0.3) (layer F.Cu) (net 5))
 (segment (start 128.27 118.872) (end 130.78851 116.35349) (width 0.3) (layer F.Cu) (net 6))
 (segment (start 125.222 115.824) (end 122.936 115.824) (width 0.3) (layer F.Cu) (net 6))
 (segment (start 128.27 118.872) (end 125.222 115.824) (width 0.3) (layer F.Cu) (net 6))
 (segment (start 128.964707 107.710001) (end 127.060001 107.710001) (width 0.3) (layer F.Cu) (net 6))
 (segment (start 130.78851 109.533804) (end 128.964707 107.710001) (width 0.3) (layer F.Cu) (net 6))
 (segment (start 127.060001 107.710001) (end 125.86 106.51) (width 0.3) (layer F.Cu) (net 6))
 (segment (start 130.78851 116.35349) (end 130.78851 109.533804) (width 0.3) (layer F.Cu) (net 6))
 (segment (start 127.605 110.236) (end 129.951 110.236) (width 0.3) (layer F.Cu) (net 1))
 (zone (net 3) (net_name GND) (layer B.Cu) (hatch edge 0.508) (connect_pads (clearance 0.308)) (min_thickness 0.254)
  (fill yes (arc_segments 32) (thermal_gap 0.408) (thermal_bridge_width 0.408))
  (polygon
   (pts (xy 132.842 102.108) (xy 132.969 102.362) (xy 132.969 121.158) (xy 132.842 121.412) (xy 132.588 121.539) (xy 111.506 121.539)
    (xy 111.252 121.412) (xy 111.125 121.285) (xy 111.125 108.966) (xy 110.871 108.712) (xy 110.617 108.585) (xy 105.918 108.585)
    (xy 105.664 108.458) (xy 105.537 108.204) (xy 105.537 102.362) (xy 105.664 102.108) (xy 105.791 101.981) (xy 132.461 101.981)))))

